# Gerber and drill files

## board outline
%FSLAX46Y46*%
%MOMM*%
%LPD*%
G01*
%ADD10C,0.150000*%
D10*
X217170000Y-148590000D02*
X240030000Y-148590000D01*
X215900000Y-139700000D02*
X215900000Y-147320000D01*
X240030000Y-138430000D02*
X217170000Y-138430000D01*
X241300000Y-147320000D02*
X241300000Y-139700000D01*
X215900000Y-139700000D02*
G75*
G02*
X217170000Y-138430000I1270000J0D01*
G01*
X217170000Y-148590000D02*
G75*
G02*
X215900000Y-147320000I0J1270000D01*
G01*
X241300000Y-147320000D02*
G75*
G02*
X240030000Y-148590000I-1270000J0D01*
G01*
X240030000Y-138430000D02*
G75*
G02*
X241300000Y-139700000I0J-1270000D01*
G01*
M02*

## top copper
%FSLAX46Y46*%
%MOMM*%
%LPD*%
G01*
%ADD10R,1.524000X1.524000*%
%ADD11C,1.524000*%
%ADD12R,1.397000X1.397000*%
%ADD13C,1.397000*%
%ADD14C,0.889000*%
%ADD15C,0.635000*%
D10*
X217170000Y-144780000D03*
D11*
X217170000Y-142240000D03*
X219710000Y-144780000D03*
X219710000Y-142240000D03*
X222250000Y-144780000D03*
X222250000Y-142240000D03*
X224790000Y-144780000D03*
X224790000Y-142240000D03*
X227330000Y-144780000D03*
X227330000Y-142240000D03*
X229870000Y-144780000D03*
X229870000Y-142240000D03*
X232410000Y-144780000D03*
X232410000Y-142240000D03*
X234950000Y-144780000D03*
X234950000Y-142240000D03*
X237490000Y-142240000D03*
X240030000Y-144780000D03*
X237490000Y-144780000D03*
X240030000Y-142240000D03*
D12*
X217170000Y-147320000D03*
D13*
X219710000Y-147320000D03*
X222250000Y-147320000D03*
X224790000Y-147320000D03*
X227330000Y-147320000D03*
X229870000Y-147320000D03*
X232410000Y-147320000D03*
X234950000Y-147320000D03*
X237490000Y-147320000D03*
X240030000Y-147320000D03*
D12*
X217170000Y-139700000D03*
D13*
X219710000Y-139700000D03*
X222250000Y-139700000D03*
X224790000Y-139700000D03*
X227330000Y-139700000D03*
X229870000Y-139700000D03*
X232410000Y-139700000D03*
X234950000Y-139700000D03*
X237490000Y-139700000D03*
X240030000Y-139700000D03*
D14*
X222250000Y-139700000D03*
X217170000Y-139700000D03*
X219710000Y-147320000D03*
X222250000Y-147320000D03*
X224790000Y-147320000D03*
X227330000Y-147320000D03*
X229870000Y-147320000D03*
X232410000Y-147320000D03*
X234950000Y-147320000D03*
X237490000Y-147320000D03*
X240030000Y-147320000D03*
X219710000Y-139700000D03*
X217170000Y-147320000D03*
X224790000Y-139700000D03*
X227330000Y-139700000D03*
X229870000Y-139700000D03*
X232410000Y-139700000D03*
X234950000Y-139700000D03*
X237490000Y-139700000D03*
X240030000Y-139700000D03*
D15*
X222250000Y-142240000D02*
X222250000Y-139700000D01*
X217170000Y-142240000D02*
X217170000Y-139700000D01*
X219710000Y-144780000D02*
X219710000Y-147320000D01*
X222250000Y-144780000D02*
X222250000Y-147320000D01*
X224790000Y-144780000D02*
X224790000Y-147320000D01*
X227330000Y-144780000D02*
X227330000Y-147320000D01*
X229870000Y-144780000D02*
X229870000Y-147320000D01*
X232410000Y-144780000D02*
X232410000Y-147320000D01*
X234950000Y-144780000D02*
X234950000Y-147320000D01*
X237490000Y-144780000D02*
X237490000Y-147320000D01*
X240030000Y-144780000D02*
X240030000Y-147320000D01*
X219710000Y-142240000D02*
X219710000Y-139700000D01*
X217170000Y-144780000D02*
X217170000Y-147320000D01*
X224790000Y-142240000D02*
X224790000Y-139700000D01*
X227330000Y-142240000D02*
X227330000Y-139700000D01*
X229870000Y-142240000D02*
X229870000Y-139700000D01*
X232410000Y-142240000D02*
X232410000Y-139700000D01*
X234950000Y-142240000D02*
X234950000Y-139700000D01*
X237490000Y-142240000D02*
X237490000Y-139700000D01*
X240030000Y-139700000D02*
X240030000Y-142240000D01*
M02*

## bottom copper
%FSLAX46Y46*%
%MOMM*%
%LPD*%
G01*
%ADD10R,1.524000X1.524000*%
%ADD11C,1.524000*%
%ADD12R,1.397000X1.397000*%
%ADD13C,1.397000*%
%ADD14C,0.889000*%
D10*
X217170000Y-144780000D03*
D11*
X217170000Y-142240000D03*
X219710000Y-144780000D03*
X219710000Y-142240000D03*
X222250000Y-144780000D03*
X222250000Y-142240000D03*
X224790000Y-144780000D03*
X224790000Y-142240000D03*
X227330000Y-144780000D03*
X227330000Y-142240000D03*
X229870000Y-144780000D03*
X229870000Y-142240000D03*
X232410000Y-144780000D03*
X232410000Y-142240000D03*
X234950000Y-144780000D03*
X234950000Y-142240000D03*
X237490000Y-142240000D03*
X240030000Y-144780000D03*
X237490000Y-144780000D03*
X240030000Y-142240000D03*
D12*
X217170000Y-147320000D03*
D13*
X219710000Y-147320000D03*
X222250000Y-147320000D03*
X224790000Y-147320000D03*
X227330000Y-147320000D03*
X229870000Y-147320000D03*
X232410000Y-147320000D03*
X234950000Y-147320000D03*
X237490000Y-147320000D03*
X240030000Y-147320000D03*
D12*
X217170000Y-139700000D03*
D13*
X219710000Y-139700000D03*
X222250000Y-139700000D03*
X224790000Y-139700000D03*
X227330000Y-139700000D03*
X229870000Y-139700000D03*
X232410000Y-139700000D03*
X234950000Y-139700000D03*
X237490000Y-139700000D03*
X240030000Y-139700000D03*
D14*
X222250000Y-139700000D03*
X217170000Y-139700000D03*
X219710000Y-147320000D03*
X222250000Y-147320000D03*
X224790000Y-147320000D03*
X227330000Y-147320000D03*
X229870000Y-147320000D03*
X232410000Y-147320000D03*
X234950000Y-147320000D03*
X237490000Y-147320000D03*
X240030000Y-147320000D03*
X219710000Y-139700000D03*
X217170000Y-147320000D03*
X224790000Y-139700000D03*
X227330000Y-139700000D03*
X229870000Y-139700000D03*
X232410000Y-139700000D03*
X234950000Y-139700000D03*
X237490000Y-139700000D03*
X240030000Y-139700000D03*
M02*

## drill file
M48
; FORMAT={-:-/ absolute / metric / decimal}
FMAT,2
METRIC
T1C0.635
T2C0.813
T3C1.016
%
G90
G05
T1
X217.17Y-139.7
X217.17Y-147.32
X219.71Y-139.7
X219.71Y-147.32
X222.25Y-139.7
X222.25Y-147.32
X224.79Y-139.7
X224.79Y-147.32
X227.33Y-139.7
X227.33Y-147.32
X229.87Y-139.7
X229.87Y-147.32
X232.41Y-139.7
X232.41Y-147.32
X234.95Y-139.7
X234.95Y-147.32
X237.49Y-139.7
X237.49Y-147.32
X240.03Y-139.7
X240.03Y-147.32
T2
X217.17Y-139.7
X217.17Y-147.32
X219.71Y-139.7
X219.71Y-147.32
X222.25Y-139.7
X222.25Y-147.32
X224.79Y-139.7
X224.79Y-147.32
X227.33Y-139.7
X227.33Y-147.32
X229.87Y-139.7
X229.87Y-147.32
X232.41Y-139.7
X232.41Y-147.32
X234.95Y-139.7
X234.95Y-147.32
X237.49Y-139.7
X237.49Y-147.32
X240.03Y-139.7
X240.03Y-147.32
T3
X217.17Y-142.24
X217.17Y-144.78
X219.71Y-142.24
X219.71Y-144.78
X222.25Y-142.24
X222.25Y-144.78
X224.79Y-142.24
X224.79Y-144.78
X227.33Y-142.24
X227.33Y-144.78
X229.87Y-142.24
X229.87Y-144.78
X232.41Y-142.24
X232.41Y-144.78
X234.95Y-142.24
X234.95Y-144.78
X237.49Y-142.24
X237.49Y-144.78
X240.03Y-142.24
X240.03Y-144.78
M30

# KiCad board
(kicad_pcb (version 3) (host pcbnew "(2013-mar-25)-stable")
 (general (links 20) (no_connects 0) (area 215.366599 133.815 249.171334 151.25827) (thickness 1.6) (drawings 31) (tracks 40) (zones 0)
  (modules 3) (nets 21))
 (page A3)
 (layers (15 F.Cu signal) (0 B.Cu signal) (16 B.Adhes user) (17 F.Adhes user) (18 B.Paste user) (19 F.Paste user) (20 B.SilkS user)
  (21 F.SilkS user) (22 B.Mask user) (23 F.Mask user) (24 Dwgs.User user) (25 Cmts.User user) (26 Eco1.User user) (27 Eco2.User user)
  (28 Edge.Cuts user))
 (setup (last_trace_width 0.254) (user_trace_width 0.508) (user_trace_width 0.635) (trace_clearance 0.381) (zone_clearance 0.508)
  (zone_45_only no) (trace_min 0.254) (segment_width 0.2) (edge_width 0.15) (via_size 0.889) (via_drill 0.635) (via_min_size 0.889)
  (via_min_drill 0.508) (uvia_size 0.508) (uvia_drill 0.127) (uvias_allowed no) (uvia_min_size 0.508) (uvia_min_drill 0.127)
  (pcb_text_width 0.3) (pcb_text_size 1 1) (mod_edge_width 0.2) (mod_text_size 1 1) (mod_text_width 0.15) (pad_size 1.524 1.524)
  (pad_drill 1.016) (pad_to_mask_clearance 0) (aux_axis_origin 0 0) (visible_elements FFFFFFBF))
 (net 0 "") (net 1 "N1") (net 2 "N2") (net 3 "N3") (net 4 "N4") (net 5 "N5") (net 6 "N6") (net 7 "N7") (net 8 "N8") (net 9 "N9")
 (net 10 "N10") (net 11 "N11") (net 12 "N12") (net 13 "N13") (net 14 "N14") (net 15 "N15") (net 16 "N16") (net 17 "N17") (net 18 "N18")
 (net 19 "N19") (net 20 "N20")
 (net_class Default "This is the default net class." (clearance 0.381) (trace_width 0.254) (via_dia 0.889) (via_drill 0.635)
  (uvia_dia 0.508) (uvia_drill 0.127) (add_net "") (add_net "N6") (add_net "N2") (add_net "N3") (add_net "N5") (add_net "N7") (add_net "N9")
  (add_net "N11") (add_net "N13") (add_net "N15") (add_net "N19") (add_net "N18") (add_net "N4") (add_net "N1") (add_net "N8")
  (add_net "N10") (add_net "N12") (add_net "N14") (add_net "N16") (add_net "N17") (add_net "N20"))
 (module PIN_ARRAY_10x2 (layer F.Cu) (at 228.6 143.51)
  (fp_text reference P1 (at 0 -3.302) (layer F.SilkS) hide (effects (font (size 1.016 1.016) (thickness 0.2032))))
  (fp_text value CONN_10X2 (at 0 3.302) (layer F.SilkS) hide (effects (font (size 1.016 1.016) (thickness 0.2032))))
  (pad 1 thru_hole rect (at -11.43 1.27) (size 1.524 1.524) (drill 1.016) (layers *.Cu *.Mask F.SilkS) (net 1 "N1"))
  (pad 2 thru_hole circle (at -11.43 -1.27) (size 1.524 1.524) (drill 1.016) (layers *.Cu *.Mask F.SilkS) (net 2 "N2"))
  (pad 3 thru_hole circle (at -8.89 1.27) (size 1.524 1.524) (drill 1.016) (layers *.Cu *.Mask F.SilkS) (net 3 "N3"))
  (pad 4 thru_hole circle (at -8.89 -1.27) (size 1.524 1.524) (drill 1.016) (layers *.Cu *.Mask F.SilkS) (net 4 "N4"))
  (pad 5 thru_hole circle (at -6.35 1.27) (size 1.524 1.524) (drill 1.016) (layers *.Cu *.Mask F.SilkS) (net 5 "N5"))
  (pad 6 thru_hole circle (at -6.35 -1.27) (size 1.524 1.524) (drill 1.016) (layers *.Cu *.Mask F.SilkS) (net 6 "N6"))
  (pad 7 thru_hole circle (at -3.81 1.27) (size 1.524 1.524) (drill 1.016) (layers *.Cu *.Mask F.SilkS) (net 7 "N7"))
  (pad 8 thru_hole circle (at -3.81 -1.27) (size 1.524 1.524) (drill 1.016) (layers *.Cu *.Mask F.SilkS) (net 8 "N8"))
  (pad 9 thru_hole circle (at -1.27 1.27) (size 1.524 1.524) (drill 1.016) (layers *.Cu *.Mask F.SilkS) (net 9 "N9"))
  (pad 10 thru_hole circle (at -1.27 -1.27) (size 1.524 1.524) (drill 1.016) (layers *.Cu *.Mask F.SilkS) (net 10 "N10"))
  (pad 11 thru_hole circle (at 1.27 1.27) (size 1.524 1.524) (drill 1.016) (layers *.Cu *.Mask F.SilkS) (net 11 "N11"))
  (pad 12 thru_hole circle (at 1.27 -1.27) (size 1.524 1.524) (drill 1.016) (layers *.Cu *.Mask F.SilkS) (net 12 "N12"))
  (pad 13 thru_hole circle (at 3.81 1.27) (size 1.524 1.524) (drill 1.016) (layers *.Cu *.Mask F.SilkS) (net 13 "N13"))
  (pad 14 thru_hole circle (at 3.81 -1.27) (size 1.524 1.524) (drill 1.016) (layers *.Cu *.Mask F.SilkS) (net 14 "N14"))
  (pad 15 thru_hole circle (at 6.35 1.27) (size 1.524 1.524) (drill 1.016) (layers *.Cu *.Mask F.SilkS) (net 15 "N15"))
  (pad 16 thru_hole circle (at 6.35 -1.27) (size 1.524 1.524) (drill 1.016) (layers *.Cu *.Mask F.SilkS) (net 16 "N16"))
  (pad 18 thru_hole circle (at 8.89 -1.27) (size 1.524 1.524) (drill 1.016) (layers *.Cu F.SilkS B.Mask) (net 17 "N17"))
  (pad 19 thru_hole circle (at 11.43 1.27) (size 1.524 1.524) (drill 1.016) (layers *.Cu F.SilkS B.Mask) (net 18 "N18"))
  (pad 17 thru_hole circle (at 8.89 1.27) (size 1.524 1.524) (drill 1.016) (layers *.Cu F.SilkS B.Mask) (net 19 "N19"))
  (pad 20 thru_hole circle (at 11.43 -1.27) (size 1.524 1.524) (drill 1.016) (layers *.Cu F.SilkS B.Mask) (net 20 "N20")))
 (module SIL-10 (layer B.Cu) (at 228.6 147.32)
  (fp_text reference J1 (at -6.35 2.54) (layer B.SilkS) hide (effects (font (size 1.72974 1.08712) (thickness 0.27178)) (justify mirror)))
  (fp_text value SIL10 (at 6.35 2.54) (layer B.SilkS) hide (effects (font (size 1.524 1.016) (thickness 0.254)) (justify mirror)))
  (pad 1 thru_hole rect (at -11.43 0) (size 1.397 1.397) (drill 0.8128) (layers *.Cu *.Mask B.SilkS) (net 1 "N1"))
  (pad 2 thru_hole circle (at -8.89 0) (size 1.397 1.397) (drill 0.8128) (layers *.Cu *.Mask B.SilkS) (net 3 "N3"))
  (pad 3 thru_hole circle (at -6.35 0) (size 1.397 1.397) (drill 0.8128) (layers *.Cu *.Mask B.SilkS) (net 5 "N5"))
  (pad 4 thru_hole circle (at -3.81 0) (size 1.397 1.397) (drill 0.8128) (layers *.Cu *.Mask B.SilkS) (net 7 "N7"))
  (pad 5 thru_hole circle (at -1.27 0) (size 1.397 1.397) (drill 0.8128) (layers *.Cu *.Mask B.SilkS) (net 9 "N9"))
  (pad 6 thru_hole circle (at 1.27 0) (size 1.397 1.397) (drill 0.8128) (layers *.Cu *.Mask B.SilkS) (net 11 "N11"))
  (pad 7 thru_hole circle (at 3.81 0) (size 1.397 1.397) (drill 0.8128) (layers *.Cu *.Mask B.SilkS) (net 13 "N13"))
  (pad 8 thru_hole circle (at 6.35 0) (size 1.397 1.397) (drill 0.8128) (layers *.Cu *.Mask B.SilkS) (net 15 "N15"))
  (pad 9 thru_hole circle (at 8.89 0) (size 1.397 1.397) (drill 0.8128) (layers *.Cu *.Mask B.SilkS) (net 19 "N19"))
  (pad 10 thru_hole circle (at 11.43 0) (size 1.397 1.397) (drill 0.8128) (layers *.Cu *.Mask B.SilkS) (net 18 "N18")))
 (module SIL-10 (layer B.Cu) (at 228.6 139.7)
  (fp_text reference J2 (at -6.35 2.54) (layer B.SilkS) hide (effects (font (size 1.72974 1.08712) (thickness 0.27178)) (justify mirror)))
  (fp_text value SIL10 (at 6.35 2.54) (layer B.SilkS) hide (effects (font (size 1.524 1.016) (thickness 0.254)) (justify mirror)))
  (pad 1 thru_hole rect (at -11.43 0) (size 1.397 1.397) (drill 0.8128) (layers *.Cu *.Mask B.SilkS) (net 2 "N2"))
  (pad 2 thru_hole circle (at -8.89 0) (size 1.397 1.397) (drill 0.8128) (layers *.Cu *.Mask B.SilkS) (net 4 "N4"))
  (pad 3 thru_hole circle (at -6.35 0) (size 1.397 1.397) (drill 0.8128) (layers *.Cu *.Mask B.SilkS) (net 6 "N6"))
  (pad 4 thru_hole circle (at -3.81 0) (size 1.397 1.397) (drill 0.8128) (layers *.Cu *.Mask B.SilkS) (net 8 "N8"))
  (pad 5 thru_hole circle (at -1.27 0) (size 1.397 1.397) (drill 0.8128) (layers *.Cu *.Mask B.SilkS) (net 10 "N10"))
  (pad 6 thru_hole circle (at 1.27 0) (size 1.397 1.397) (drill 0.8128) (layers *.Cu *.Mask B.SilkS) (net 12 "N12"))
  (pad 7 thru_hole circle (at 3.81 0) (size 1.397 1.397) (drill 0.8128) (layers *.Cu *.Mask B.SilkS) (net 14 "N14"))
  (pad 8 thru_hole circle (at 6.35 0) (size 1.397 1.397) (drill 0.8128) (layers *.Cu *.Mask B.SilkS) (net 16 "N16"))
  (pad 9 thru_hole circle (at 8.89 0) (size 1.397 1.397) (drill 0.8128) (layers *.Cu *.Mask B.SilkS) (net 17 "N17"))
  (pad 10 thru_hole circle (at 11.43 0) (size 1.397 1.397) (drill 0.8128) (layers *.Cu *.Mask B.SilkS) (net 20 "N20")))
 (gr_line (start 217.17 148.59) (end 240.03 148.59) (angle 90) (layer Edge.Cuts) (width 0.15))
 (gr_line (start 215.9 139.7) (end 215.9 147.32) (angle 90) (layer Edge.Cuts) (width 0.15))
 (gr_line (start 240.03 138.43) (end 217.17 138.43) (angle 90) (layer Edge.Cuts) (width 0.15))
 (gr_line (start 241.3 147.32) (end 241.3 139.7) (angle 90) (layer Edge.Cuts) (width 0.15))
 (gr_arc (start 217.17 139.7) (end 215.9 139.7) (angle 90) (layer Edge.Cuts) (width 0.15))
 (gr_arc (start 217.17 147.32) (end 217.17 148.59) (angle 90) (layer Edge.Cuts) (width 0.15))
 (gr_arc (start 240.03 147.32) (end 241.3 147.32) (angle 90) (layer Edge.Cuts) (width 0.15))
 (gr_arc (start 240.03 139.7) (end 240.03 138.43) (angle 90) (layer Edge.Cuts) (width 0.15))
 (segment (start 222.25 142.24) (end 222.25 139.7) (width 0.635) (layer F.Cu) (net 6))
 (via (at 222.25 139.7) (size 0.889) (layers F.Cu B.Cu) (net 6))
 (segment (start 217.17 142.24) (end 217.17 139.7) (width 0.635) (layer F.Cu) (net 2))
 (via (at 217.17 139.7) (size 0.889) (layers F.Cu B.Cu) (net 2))
 (segment (start 219.71 144.78) (end 219.71 147.32) (width 0.635) (layer F.Cu) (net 3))
 (via (at 219.71 147.32) (size 0.889) (layers F.Cu B.Cu) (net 3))
 (segment (start 222.25 144.78) (end 222.25 147.32) (width 0.635) (layer F.Cu) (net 5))
 (via (at 222.25 147.32) (size 0.889) (layers F.Cu B.Cu) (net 5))
 (segment (start 224.79 144.78) (end 224.79 147.32) (width 0.635) (layer F.Cu) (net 7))
 (via (at 224.79 147.32) (size 0.889) (layers F.Cu B.Cu) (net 7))
 (segment (start 227.33 144.78) (end 227.33 147.32) (width 0.635) (layer F.Cu) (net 9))
 (via (at 227.33 147.32) (size 0.889) (layers F.Cu B.Cu) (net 9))
 (segment (start 229.87 144.78) (end 229.87 147.32) (width 0.635) (layer F.Cu) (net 11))
 (via (at 229.87 147.32) (size 0.889) (layers F.Cu B.Cu) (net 11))
 (segment (start 232.41 144.78) (end 232.41 147.32) (width 0.635) (layer F.Cu) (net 13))
 (via (at 232.41 147.32) (size 0.889) (layers F.Cu B.Cu) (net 13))
 (segment (start 234.95 144.78) (end 234.95 147.32) (width 0.635) (layer F.Cu) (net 15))
 (via (at 234.95 147.32) (size 0.889) (layers F.Cu B.Cu) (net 15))
 (segment (start 237.49 144.78) (end 237.49 147.32) (width 0.635) (layer F.Cu) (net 19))
 (via (at 237.49 147.32) (size 0.889) (layers F.Cu B.Cu) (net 19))
 (segment (start 240.03 144.78) (end 240.03 147.32) (width 0.635) (layer F.Cu) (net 18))
 (via (at 240.03 147.32) (size 0.889) (layers F.Cu B.Cu) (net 18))
 (segment (start 219.71 142.24) (end 219.71 139.7) (width 0.635) (layer F.Cu) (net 4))
 (via (at 219.71 139.7) (size 0.889) (layers F.Cu B.Cu) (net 4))
 (segment (start 217.17 144.78) (end 217.17 147.32) (width 0.635) (layer F.Cu) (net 1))
 (via (at 217.17 147.32) (size 0.889) (layers F.Cu B.Cu) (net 1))
 (segment (start 224.79 142.24) (end 224.79 139.7) (width 0.635) (layer F.Cu) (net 8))
 (via (at 224.79 139.7) (size 0.889) (layers F.Cu B.Cu) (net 8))
 (segment (start 227.33 142.24) (end 227.33 139.7) (width 0.635) (layer F.Cu) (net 10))
 (via (at 227.33 139.7) (size 0.889) (layers F.Cu B.Cu) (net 10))
 (segment (start 229.87 142.24) (end 229.87 139.7) (width 0.635) (layer F.Cu) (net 12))
 (via (at 229.87 139.7) (size 0.889) (layers F.Cu B.Cu) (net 12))
 (segment (start 232.41 142.24) (end 232.41 139.7) (width 0.635) (layer F.Cu) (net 14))
 (via (at 232.41 139.7) (size 0.889) (layers F.Cu B.Cu) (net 14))
 (segment (start 234.95 142.24) (end 234.95 139.7) (width 0.635) (layer F.Cu) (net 16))
 (via (at 234.95 139.7) (size 0.889) (layers F.Cu B.Cu) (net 16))
 (segment (start 237.49 142.24) (end 237.49 139.7) (width 0.635) (layer F.Cu) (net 17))
 (via (at 237.49 139.7) (size 0.889) (layers F.Cu B.Cu) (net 17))
 (via (at 240.03 139.7) (size 0.889) (layers F.Cu B.Cu) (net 20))
 (segment (start 240.03 139.7) (end 240.03 142.24) (width 0.635) (layer F.Cu) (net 20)))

